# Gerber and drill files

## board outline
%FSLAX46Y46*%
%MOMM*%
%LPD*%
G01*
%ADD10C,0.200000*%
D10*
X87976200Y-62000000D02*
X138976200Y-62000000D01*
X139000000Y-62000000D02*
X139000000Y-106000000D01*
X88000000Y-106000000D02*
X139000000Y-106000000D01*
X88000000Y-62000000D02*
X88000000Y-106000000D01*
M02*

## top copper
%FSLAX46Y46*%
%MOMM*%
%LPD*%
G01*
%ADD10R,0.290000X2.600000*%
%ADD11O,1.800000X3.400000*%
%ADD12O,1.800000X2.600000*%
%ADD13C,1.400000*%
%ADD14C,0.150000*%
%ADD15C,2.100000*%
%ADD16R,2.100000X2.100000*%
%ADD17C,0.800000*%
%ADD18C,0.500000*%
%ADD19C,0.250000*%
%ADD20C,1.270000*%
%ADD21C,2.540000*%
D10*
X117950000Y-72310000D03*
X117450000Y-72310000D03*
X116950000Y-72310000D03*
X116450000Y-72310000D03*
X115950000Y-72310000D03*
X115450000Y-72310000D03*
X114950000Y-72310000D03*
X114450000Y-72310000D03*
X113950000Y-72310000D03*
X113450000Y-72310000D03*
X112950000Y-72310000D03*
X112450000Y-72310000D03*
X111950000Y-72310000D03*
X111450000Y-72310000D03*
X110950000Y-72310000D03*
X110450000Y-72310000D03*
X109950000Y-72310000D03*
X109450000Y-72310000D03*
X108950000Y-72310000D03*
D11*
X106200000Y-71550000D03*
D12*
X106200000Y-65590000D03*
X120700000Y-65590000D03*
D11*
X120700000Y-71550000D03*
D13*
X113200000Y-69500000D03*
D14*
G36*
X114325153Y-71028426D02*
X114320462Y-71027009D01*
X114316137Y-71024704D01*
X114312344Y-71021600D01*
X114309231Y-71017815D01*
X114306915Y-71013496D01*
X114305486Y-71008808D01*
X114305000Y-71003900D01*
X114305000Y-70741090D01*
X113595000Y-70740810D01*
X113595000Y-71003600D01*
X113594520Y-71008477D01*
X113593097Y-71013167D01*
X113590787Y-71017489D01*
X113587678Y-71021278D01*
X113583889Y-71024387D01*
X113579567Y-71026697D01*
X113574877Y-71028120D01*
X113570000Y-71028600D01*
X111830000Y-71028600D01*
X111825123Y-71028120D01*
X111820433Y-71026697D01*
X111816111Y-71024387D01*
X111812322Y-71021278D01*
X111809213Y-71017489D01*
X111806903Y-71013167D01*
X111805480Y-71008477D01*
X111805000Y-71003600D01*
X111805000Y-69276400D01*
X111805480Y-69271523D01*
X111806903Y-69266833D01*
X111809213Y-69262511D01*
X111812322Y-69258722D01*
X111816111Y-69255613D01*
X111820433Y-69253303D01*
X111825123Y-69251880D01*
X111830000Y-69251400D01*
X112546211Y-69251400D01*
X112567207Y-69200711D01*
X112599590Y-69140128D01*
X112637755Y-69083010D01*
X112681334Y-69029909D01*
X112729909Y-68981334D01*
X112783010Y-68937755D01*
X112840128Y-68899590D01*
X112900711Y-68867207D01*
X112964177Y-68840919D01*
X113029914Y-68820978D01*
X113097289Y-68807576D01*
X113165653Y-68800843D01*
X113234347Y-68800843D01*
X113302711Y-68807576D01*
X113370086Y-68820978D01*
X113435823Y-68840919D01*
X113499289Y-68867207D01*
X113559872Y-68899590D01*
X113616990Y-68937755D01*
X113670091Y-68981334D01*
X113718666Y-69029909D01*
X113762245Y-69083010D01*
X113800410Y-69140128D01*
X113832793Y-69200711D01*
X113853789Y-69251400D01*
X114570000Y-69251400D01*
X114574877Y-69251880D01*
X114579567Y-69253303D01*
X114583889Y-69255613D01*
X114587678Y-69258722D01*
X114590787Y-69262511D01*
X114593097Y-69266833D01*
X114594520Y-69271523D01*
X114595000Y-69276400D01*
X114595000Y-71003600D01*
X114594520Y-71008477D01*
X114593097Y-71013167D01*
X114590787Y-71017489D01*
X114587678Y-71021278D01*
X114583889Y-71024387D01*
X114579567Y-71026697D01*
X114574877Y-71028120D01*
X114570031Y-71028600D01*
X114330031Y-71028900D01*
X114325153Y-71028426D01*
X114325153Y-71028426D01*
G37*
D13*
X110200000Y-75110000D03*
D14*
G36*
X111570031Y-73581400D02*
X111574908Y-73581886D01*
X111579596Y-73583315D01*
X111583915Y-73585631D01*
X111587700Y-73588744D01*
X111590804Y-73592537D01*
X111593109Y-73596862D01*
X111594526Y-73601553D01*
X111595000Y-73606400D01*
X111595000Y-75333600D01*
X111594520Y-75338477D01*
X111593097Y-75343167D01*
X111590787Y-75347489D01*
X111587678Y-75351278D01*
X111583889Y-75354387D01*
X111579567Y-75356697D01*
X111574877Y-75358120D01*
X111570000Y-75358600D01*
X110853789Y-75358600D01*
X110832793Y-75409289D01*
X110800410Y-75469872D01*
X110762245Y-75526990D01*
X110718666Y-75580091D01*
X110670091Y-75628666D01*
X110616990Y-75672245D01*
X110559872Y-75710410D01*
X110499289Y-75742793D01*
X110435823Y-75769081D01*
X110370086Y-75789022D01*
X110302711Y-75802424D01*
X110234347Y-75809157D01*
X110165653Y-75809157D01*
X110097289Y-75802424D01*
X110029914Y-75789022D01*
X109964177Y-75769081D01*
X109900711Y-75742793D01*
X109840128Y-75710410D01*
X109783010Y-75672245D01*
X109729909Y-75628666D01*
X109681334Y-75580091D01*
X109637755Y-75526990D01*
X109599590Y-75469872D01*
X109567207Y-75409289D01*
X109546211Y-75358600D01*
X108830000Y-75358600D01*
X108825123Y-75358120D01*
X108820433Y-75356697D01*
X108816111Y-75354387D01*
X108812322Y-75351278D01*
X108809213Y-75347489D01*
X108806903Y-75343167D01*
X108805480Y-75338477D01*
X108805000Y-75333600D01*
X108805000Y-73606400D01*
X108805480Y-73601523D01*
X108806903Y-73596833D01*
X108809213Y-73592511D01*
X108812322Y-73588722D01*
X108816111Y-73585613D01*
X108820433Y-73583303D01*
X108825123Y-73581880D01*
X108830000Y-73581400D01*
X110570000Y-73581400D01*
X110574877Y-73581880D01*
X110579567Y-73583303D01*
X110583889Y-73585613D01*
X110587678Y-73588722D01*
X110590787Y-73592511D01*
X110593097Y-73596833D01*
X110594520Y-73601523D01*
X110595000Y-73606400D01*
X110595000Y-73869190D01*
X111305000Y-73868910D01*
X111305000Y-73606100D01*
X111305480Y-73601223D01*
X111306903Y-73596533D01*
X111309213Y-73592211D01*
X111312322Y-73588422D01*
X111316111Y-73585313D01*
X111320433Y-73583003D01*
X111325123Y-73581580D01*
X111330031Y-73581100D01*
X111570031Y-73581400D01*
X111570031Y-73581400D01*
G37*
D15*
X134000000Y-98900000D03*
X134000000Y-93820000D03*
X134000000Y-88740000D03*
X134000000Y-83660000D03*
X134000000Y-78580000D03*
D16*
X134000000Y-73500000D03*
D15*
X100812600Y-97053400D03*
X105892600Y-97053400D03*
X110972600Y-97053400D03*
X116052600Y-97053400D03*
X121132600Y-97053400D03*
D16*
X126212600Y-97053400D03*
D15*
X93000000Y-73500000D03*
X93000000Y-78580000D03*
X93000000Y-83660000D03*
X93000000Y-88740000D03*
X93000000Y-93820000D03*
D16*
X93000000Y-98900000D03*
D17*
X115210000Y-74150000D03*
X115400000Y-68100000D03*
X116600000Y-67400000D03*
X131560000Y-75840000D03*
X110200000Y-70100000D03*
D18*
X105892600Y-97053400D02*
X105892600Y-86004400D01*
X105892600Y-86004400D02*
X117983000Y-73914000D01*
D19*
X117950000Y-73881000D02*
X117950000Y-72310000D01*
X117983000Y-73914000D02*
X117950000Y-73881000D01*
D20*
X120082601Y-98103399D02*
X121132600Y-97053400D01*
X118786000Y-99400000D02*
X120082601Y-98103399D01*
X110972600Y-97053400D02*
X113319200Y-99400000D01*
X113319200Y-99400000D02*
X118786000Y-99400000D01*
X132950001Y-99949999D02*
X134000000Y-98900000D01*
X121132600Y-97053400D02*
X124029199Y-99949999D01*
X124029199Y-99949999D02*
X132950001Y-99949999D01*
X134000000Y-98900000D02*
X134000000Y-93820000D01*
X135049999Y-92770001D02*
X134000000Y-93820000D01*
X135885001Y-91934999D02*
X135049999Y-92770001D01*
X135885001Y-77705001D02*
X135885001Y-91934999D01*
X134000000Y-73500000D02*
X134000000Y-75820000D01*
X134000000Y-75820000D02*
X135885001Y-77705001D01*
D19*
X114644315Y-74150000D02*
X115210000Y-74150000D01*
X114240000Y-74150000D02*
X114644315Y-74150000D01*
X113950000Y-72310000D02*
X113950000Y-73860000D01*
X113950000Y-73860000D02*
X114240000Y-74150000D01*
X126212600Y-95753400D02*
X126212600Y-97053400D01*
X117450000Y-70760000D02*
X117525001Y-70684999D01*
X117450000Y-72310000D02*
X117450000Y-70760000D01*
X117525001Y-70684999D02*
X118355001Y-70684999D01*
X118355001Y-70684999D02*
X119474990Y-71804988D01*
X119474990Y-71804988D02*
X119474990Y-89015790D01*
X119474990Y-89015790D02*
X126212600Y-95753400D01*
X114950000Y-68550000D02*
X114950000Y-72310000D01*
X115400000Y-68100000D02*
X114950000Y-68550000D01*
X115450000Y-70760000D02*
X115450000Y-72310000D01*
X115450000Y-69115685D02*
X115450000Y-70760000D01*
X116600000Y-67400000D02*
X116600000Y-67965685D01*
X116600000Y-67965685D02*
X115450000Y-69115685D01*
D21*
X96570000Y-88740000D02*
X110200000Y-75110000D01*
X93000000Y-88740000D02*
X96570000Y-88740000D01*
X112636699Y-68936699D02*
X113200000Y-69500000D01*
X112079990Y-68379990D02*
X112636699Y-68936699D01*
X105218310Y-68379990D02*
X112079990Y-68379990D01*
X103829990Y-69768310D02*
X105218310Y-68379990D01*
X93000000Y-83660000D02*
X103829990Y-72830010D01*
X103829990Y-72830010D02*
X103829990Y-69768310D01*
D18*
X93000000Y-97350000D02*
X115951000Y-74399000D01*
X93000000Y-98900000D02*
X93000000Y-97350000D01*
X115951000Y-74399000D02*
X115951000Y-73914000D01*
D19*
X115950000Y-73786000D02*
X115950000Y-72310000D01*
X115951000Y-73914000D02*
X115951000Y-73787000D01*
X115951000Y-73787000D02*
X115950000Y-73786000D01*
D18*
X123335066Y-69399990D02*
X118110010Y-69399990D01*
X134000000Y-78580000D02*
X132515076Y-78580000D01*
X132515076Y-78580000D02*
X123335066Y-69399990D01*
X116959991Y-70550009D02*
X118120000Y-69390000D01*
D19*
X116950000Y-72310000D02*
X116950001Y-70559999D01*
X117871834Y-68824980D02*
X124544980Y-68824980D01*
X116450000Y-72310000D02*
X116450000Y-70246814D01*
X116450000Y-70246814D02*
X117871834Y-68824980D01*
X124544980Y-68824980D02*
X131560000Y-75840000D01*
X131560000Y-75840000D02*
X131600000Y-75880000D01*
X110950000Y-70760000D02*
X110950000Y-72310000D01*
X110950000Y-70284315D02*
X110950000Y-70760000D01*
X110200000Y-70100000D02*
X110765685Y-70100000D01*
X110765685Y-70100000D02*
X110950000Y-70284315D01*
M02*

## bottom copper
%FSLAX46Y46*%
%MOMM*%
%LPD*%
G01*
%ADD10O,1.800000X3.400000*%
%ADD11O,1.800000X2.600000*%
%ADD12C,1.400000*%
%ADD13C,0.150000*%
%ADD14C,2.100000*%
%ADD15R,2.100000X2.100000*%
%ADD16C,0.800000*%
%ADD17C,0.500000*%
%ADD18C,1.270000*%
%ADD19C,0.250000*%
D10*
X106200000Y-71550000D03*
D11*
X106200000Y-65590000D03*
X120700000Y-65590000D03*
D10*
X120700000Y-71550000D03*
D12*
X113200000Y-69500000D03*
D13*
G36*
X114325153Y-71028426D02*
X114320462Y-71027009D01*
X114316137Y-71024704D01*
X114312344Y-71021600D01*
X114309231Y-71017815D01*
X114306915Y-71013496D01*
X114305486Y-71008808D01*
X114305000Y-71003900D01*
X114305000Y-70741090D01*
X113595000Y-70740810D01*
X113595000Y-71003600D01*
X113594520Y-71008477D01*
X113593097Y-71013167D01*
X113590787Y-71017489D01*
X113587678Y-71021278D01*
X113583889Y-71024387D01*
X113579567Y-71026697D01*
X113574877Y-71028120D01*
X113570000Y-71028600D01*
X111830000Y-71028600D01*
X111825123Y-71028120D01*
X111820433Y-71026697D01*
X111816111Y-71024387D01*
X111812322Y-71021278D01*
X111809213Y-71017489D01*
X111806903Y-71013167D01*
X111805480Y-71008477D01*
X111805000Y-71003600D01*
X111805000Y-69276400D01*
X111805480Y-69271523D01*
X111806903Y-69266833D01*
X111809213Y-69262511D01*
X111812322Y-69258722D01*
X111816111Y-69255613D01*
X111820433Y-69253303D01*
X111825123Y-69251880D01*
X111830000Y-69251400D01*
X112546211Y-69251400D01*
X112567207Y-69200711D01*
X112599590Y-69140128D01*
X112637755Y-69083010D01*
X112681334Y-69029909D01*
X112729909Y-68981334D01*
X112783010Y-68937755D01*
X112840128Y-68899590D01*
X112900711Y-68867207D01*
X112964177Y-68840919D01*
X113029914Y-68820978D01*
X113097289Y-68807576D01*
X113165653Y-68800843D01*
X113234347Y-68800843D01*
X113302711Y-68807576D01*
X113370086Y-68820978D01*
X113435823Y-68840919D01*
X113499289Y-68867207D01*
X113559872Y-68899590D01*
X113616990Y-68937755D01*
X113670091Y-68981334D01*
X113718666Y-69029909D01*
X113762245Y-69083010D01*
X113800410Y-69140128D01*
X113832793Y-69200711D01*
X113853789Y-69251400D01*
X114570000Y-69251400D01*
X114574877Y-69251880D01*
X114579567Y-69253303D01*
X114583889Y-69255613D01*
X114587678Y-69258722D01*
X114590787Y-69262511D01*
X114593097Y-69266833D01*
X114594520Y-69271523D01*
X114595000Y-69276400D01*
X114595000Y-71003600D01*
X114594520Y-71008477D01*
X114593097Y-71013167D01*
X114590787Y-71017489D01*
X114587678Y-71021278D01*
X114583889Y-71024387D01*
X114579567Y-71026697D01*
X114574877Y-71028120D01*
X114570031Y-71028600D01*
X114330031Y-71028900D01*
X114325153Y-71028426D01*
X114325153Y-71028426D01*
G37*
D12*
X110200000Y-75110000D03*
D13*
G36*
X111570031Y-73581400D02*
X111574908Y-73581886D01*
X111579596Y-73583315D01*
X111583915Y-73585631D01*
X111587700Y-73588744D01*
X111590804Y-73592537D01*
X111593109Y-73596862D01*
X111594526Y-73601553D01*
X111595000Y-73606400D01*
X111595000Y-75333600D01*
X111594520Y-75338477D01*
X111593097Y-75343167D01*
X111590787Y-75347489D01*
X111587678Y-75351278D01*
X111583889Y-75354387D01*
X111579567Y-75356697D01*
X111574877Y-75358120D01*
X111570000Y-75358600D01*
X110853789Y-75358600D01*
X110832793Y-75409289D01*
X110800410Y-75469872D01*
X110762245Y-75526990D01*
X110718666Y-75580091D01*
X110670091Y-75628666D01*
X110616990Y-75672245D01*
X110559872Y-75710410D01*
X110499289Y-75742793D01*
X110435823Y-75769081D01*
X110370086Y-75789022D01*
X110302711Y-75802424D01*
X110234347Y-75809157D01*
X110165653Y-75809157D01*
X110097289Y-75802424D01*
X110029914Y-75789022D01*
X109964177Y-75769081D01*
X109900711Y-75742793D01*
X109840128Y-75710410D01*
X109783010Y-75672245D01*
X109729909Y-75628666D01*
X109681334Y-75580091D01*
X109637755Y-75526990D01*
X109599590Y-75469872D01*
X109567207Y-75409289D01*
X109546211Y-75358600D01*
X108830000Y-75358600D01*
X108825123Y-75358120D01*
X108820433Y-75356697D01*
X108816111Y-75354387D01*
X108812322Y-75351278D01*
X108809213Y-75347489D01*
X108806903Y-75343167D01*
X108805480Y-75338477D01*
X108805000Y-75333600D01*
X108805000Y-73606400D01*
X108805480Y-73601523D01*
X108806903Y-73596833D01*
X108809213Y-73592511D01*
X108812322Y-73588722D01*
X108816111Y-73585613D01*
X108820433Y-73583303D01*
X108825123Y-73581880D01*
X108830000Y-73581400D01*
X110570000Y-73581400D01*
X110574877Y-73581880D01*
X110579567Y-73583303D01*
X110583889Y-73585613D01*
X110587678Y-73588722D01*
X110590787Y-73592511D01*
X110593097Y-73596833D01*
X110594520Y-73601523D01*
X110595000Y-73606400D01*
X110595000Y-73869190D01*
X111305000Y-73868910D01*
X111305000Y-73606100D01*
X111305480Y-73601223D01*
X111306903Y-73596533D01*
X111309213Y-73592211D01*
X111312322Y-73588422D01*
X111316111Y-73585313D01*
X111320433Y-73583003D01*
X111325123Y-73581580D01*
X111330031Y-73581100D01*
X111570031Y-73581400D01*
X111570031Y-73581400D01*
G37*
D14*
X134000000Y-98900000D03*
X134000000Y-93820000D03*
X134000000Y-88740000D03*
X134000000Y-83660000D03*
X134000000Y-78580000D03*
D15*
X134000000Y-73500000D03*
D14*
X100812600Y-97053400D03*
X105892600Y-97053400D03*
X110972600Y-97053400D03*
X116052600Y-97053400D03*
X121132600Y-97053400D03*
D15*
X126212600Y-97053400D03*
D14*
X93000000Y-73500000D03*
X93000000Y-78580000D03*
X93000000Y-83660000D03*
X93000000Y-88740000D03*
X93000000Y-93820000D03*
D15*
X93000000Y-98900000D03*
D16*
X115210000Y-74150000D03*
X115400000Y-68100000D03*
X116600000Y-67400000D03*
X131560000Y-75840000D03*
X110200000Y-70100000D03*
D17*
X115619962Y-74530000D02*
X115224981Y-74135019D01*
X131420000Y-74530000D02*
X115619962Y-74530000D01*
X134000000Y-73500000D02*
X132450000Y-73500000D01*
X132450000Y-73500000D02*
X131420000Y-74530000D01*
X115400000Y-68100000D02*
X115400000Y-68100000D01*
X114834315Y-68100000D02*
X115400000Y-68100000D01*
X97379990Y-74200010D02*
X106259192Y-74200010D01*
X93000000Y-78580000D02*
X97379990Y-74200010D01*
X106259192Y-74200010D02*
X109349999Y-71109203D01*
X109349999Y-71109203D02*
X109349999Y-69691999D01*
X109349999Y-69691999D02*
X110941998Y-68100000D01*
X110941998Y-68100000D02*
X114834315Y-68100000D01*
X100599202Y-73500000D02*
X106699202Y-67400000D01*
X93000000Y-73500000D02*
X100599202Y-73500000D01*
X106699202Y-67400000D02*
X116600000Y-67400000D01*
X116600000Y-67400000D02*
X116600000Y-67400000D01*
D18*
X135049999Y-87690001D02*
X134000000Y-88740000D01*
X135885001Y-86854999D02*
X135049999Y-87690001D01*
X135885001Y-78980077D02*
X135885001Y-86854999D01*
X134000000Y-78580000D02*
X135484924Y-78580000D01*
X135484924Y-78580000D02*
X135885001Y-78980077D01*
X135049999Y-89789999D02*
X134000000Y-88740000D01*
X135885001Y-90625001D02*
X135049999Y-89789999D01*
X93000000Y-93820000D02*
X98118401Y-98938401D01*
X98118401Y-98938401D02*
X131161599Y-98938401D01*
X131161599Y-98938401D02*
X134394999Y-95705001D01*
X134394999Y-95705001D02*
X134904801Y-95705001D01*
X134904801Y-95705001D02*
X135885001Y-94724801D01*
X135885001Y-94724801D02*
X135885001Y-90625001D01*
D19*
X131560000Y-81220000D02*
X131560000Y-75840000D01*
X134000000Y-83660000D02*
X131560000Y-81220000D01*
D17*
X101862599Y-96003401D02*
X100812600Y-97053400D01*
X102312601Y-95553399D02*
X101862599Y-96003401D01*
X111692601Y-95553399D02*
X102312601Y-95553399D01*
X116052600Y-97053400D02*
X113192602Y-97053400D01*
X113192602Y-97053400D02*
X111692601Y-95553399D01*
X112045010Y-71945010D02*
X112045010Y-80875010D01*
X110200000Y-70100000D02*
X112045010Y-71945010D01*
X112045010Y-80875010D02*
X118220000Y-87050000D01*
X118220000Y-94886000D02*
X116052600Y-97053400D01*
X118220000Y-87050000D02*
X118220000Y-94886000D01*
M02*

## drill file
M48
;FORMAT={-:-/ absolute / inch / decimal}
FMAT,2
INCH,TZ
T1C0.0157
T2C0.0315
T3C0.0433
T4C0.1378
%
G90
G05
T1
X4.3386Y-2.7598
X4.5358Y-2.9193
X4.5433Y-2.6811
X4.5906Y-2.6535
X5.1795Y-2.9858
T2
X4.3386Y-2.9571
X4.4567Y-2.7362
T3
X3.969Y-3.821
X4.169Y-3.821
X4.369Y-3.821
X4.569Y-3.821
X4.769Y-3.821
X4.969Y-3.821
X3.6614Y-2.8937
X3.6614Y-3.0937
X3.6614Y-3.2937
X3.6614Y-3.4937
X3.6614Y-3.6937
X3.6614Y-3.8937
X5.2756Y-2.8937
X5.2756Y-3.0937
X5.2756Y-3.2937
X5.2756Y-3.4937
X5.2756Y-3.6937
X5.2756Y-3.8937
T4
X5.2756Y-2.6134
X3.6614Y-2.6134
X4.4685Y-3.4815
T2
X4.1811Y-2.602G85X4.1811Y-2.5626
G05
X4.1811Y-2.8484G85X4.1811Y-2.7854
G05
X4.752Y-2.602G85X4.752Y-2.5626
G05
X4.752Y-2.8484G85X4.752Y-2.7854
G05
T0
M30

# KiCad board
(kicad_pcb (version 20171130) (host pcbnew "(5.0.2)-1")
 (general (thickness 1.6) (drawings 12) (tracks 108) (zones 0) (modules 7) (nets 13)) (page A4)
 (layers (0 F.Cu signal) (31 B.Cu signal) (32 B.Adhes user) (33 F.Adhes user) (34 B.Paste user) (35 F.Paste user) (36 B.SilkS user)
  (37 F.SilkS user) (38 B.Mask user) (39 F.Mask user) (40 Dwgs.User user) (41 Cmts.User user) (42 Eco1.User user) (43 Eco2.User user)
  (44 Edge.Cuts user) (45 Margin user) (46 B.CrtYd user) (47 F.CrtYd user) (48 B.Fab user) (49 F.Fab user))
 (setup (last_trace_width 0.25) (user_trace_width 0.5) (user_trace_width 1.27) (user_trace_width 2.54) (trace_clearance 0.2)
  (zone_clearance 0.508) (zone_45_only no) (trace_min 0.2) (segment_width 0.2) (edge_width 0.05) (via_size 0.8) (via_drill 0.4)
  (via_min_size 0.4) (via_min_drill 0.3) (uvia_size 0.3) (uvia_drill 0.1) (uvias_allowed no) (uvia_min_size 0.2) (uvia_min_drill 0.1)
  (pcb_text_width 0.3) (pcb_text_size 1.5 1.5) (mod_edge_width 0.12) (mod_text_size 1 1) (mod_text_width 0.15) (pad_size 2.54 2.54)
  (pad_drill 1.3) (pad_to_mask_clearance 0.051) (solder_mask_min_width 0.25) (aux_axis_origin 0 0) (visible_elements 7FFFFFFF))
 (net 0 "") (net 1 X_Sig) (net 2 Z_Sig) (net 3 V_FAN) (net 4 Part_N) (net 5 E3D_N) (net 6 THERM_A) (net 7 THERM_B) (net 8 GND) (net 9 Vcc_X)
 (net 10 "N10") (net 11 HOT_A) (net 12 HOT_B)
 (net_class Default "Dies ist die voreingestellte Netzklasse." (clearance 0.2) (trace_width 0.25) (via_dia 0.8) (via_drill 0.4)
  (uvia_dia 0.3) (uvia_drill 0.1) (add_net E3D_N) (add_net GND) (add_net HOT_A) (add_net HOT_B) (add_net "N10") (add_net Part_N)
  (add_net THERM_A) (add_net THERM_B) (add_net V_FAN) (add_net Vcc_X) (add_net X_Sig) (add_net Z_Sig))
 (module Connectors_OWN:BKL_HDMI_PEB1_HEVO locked (layer F.Cu) (at 120.7 62 180)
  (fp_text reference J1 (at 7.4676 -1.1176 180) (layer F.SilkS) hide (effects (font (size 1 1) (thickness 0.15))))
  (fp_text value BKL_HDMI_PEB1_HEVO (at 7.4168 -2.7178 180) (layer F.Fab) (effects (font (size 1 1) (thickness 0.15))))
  (pad 19 smd rect (at 2.75 -10.31 180) (size 0.29 2.6) (layers F.Cu F.Paste F.Mask) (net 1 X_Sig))
  (pad 18 smd rect (at 3.25 -10.31 180) (size 0.29 2.6) (layers F.Cu F.Paste F.Mask) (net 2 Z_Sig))
  (pad 17 smd rect (at 3.75 -10.31 180) (size 0.29 2.6) (layers F.Cu F.Paste F.Mask) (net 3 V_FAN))
  (pad 16 smd rect (at 4.25 -10.31 180) (size 0.29 2.6) (layers F.Cu F.Paste F.Mask) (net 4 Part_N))
  (pad 15 smd rect (at 4.75 -10.31 180) (size 0.29 2.6) (layers F.Cu F.Paste F.Mask) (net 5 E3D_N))
  (pad 14 smd rect (at 5.25 -10.31 180) (size 0.29 2.6) (layers F.Cu F.Paste F.Mask) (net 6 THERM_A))
  (pad 13 smd rect (at 5.75 -10.31 180) (size 0.29 2.6) (layers F.Cu F.Paste F.Mask) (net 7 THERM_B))
  (pad "" smd rect (at 6.25 -10.31 180) (size 0.29 2.6) (layers F.Cu F.Paste F.Mask))
  (pad 11 smd rect (at 6.75 -10.31 180) (size 0.29 2.6) (layers F.Cu F.Paste F.Mask) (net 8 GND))
  (pad "" smd rect (at 7.25 -10.31 180) (size 0.29 2.6) (layers F.Cu F.Paste F.Mask))
  (pad "" smd rect (at 7.75 -10.31 180) (size 0.29 2.6) (layers F.Cu F.Paste F.Mask))
  (pad "" smd rect (at 8.25 -10.31 180) (size 0.29 2.6) (layers F.Cu F.Paste F.Mask))
  (pad "" smd rect (at 8.75 -10.31 180) (size 0.29 2.6) (layers F.Cu F.Paste F.Mask))
  (pad "" smd rect (at 9.25 -10.31 180) (size 0.29 2.6) (layers F.Cu F.Paste F.Mask))
  (pad 5 smd rect (at 9.75 -10.31 180) (size 0.29 2.6) (layers F.Cu F.Paste F.Mask) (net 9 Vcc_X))
  (pad "" smd rect (at 10.25 -10.31 180) (size 0.29 2.6) (layers F.Cu F.Paste F.Mask))
  (pad "" smd rect (at 10.75 -10.31 180) (size 0.29 2.6) (layers F.Cu F.Paste F.Mask))
  (pad "" smd rect (at 11.25 -10.31 180) (size 0.29 2.6) (layers F.Cu F.Paste F.Mask))
  (pad "" smd rect (at 11.75 -10.31 180) (size 0.29 2.6) (layers F.Cu F.Paste F.Mask))
  (pad SH thru_hole oval (at 14.5 -9.55 180) (size 1.8 3.4) (drill oval 0.8 2.4) (layers *.Cu *.Mask) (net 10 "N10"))
  (pad SH thru_hole oval (at 14.5 -3.59 180) (size 1.8 2.6) (drill oval 0.8 1.8) (layers *.Cu *.Mask) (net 10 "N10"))
  (pad SH thru_hole oval (at 0 -3.59 180) (size 1.8 2.6) (drill oval 0.8 1.8) (layers *.Cu *.Mask) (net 10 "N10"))
  (pad SH thru_hole oval (at 0 -9.55 180) (size 1.8 3.4) (drill oval 0.8 2.4) (layers *.Cu *.Mask) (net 10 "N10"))
  (pad 7 thru_hole custom (at 7.5 -7.5 180) (size 1.4 1.4) (drill 0.8) (layers *.Cu *.Mask) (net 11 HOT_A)
   (options (clearance outline) (anchor circle)) (primitives))
  (pad 1 thru_hole custom (at 10.5 -13.11) (size 1.4 1.4) (drill 0.8) (layers *.Cu *.Mask) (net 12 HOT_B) (zone_connect 0)
   (options (clearance outline) (anchor circle)) (primitives)))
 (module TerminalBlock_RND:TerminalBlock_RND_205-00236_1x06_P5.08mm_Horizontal (layer F.Cu) (at 134 73.5 270)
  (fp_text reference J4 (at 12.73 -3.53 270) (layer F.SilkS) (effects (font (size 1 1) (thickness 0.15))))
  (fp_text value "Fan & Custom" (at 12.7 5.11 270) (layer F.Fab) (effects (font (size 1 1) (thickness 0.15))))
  (pad 6 thru_hole circle (at 25.4 0 270) (size 2.1 2.1) (drill 1.1) (layers *.Cu *.Mask) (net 8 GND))
  (pad 5 thru_hole circle (at 20.32 0 270) (size 2.1 2.1) (drill 1.1) (layers *.Cu *.Mask) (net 8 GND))
  (pad 4 thru_hole circle (at 15.24 0 270) (size 2.1 2.1) (drill 1.1) (layers *.Cu *.Mask) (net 3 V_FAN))
  (pad 3 thru_hole circle (at 10.16 0 270) (size 2.1 2.1) (drill 1.1) (layers *.Cu *.Mask) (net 4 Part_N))
  (pad 2 thru_hole circle (at 5.08 0 270) (size 2.1 2.1) (drill 1.1) (layers *.Cu *.Mask) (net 3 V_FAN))
  (pad 1 thru_hole rect (at 0 0 270) (size 2.1 2.1) (drill 1.1) (layers *.Cu *.Mask) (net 8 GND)))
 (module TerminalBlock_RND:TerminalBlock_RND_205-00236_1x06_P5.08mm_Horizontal (layer F.Cu) (at 126.2126 97.0534 180)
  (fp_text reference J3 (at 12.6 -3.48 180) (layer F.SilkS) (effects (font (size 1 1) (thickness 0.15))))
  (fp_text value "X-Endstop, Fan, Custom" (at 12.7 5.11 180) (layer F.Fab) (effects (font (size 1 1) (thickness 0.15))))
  (pad 6 thru_hole circle (at 25.4 0 180) (size 2.1 2.1) (drill 1.1) (layers *.Cu *.Mask) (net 9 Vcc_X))
  (pad 5 thru_hole circle (at 20.32 0 180) (size 2.1 2.1) (drill 1.1) (layers *.Cu *.Mask) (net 1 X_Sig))
  (pad 4 thru_hole circle (at 15.24 0 180) (size 2.1 2.1) (drill 1.1) (layers *.Cu *.Mask) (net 8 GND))
  (pad 3 thru_hole circle (at 10.16 0 180) (size 2.1 2.1) (drill 1.1) (layers *.Cu *.Mask) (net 9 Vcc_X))
  (pad 2 thru_hole circle (at 5.08 0 180) (size 2.1 2.1) (drill 1.1) (layers *.Cu *.Mask) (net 8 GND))
  (pad 1 thru_hole rect (at 0 0 180) (size 2.1 2.1) (drill 1.1) (layers *.Cu *.Mask) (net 2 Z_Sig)))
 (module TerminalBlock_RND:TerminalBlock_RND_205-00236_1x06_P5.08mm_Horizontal (layer F.Cu) (at 93 98.9 90)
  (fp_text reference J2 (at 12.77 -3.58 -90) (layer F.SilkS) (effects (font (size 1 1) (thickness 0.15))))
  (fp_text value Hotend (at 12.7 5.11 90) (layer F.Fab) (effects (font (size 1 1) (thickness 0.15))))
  (pad 6 thru_hole circle (at 25.4 0 90) (size 2.1 2.1) (drill 1.1) (layers *.Cu *.Mask) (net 6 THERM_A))
  (pad 5 thru_hole circle (at 20.32 0 90) (size 2.1 2.1) (drill 1.1) (layers *.Cu *.Mask) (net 7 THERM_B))
  (pad 4 thru_hole circle (at 15.24 0 90) (size 2.1 2.1) (drill 1.1) (layers *.Cu *.Mask) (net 11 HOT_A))
  (pad 3 thru_hole circle (at 10.16 0 90) (size 2.1 2.1) (drill 1.1) (layers *.Cu *.Mask) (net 12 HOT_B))
  (pad 2 thru_hole circle (at 5.08 0 90) (size 2.1 2.1) (drill 1.1) (layers *.Cu *.Mask) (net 3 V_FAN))
  (pad 1 thru_hole rect (at 0 0 90) (size 2.1 2.1) (drill 1.1) (layers *.Cu *.Mask) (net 5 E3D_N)))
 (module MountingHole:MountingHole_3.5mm (layer F.Cu) (at 113.5 88.43)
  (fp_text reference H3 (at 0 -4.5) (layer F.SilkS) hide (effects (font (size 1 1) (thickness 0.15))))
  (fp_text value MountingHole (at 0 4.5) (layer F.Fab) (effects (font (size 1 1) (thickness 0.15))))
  (pad 1 np_thru_hole circle (at 0 0) (size 3.5 3.5) (drill 3.5) (layers *.Cu *.Mask)))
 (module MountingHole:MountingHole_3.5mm (layer F.Cu) (at 134 66.38)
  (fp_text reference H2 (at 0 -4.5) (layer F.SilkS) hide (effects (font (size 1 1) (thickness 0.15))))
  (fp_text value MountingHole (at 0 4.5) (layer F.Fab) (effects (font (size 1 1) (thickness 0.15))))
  (pad 1 np_thru_hole circle (at 0 0) (size 3.5 3.5) (drill 3.5) (layers *.Cu *.Mask)))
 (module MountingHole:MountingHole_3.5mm (layer F.Cu) (at 93 66.38)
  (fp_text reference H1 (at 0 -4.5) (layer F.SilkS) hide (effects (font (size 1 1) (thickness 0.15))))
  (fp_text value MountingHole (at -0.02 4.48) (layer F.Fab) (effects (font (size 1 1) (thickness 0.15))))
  (pad 1 np_thru_hole circle (at 0 0) (size 3.5 3.5) (drill 3.5) (layers *.Cu *.Mask)))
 (gr_line (start 87.9762 62) (end 138.9762 62) (layer Edge.Cuts) (width 0.2))
 (gr_line (start 139 62) (end 139 106) (layer Edge.Cuts) (width 0.2))
 (gr_line (start 88 106) (end 139 106) (layer Edge.Cuts) (width 0.2))
 (gr_line (start 88 62) (end 88 106) (layer Edge.Cuts) (width 0.2))
 (segment (start 105.8926 97.0534) (end 105.8926 86.0044) (width 0.5) (layer F.Cu) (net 1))
 (segment (start 105.8926 86.0044) (end 117.983 73.914) (width 0.5) (layer F.Cu) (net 1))
 (segment (start 117.95 73.881) (end 117.95 72.31) (width 0.25) (layer F.Cu) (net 1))
 (segment (start 117.983 73.914) (end 117.95 73.881) (width 0.25) (layer F.Cu) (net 1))
 (via (at 115.21 74.15) (size 0.8) (drill 0.4) (layers F.Cu B.Cu) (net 8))
 (segment (start 120.082601 98.103399) (end 121.1326 97.0534) (width 1.27) (layer F.Cu) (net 8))
 (segment (start 118.786 99.4) (end 120.082601 98.103399) (width 1.27) (layer F.Cu) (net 8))
 (segment (start 110.9726 97.0534) (end 113.3192 99.4) (width 1.27) (layer F.Cu) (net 8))
 (segment (start 113.3192 99.4) (end 118.786 99.4) (width 1.27) (layer F.Cu) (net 8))
 (segment (start 132.950001 99.949999) (end 134 98.9) (width 1.27) (layer F.Cu) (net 8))
 (segment (start 121.1326 97.0534) (end 124.029199 99.949999) (width 1.27) (layer F.Cu) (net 8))
 (segment (start 124.029199 99.949999) (end 132.950001 99.949999) (width 1.27) (layer F.Cu) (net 8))
 (segment (start 134 98.9) (end 134 93.82) (width 1.27) (layer F.Cu) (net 8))
 (segment (start 135.049999 92.770001) (end 134 93.82) (width 1.27) (layer F.Cu) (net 8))
 (segment (start 135.885001 91.934999) (end 135.049999 92.770001) (width 1.27) (layer F.Cu) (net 8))
 (segment (start 135.885001 77.705001) (end 135.885001 91.934999) (width 1.27) (layer F.Cu) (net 8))
 (segment (start 134 73.5) (end 134 75.82) (width 1.27) (layer F.Cu) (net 8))
 (segment (start 134 75.82) (end 135.885001 77.705001) (width 1.27) (layer F.Cu) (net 8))
 (segment (start 114.644315 74.15) (end 115.21 74.15) (width 0.25) (layer F.Cu) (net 8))
 (segment (start 114.24 74.15) (end 114.644315 74.15) (width 0.25) (layer F.Cu) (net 8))
 (segment (start 113.95 72.31) (end 113.95 73.86) (width 0.25) (layer F.Cu) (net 8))
 (segment (start 113.95 73.86) (end 114.24 74.15) (width 0.25) (layer F.Cu) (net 8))
 (segment (start 115.619962 74.53) (end 115.224981 74.135019) (width 0.5) (layer B.Cu) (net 8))
 (segment (start 131.42 74.53) (end 115.619962 74.53) (width 0.5) (layer B.Cu) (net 8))
 (segment (start 134 73.5) (end 132.45 73.5) (width 0.5) (layer B.Cu) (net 8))
 (segment (start 132.45 73.5) (end 131.42 74.53) (width 0.5) (layer B.Cu) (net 8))
 (segment (start 126.2126 95.7534) (end 126.2126 97.0534) (width 0.25) (layer F.Cu) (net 2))
 (segment (start 117.45 70.76) (end 117.525001 70.684999) (width 0.25) (layer F.Cu) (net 2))
 (segment (start 117.45 72.31) (end 117.45 70.76) (width 0.25) (layer F.Cu) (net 2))
 (segment (start 117.525001 70.684999) (end 118.355001 70.684999) (width 0.25) (layer F.Cu) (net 2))
 (segment (start 118.355001 70.684999) (end 119.47499 71.804988) (width 0.25) (layer F.Cu) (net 2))
 (segment (start 119.47499 71.804988) (end 119.47499 89.01579) (width 0.25) (layer F.Cu) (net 2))
 (segment (start 119.47499 89.01579) (end 126.2126 95.7534) (width 0.25) (layer F.Cu) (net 2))
 (segment (start 115.4 68.1) (end 115.4 68.1) (width 0.5) (layer B.Cu) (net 7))
 (via (at 115.4 68.1) (size 0.8) (drill 0.4) (layers F.Cu B.Cu) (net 7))
 (segment (start 114.95 68.55) (end 114.95 72.31) (width 0.25) (layer F.Cu) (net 7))
 (segment (start 115.4 68.1) (end 114.95 68.55) (width 0.25) (layer F.Cu) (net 7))
 (segment (start 114.834315 68.1) (end 115.4 68.1) (width 0.5) (layer B.Cu) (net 7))
 (segment (start 97.37999 74.20001) (end 106.259192 74.20001) (width 0.5) (layer B.Cu) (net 7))
 (segment (start 93 78.58) (end 97.37999 74.20001) (width 0.5) (layer B.Cu) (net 7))
 (segment (start 106.259192 74.20001) (end 109.349999 71.109203) (width 0.5) (layer B.Cu) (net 7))
 (segment (start 109.349999 71.109203) (end 109.349999 69.691999) (width 0.5) (layer B.Cu) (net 7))
 (segment (start 109.349999 69.691999) (end 110.941998 68.1) (width 0.5) (layer B.Cu) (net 7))
 (segment (start 110.941998 68.1) (end 114.834315 68.1) (width 0.5) (layer B.Cu) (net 7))
 (segment (start 100.599202 73.5) (end 106.699202 67.4) (width 0.5) (layer B.Cu) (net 6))
 (segment (start 93 73.5) (end 100.599202 73.5) (width 0.5) (layer B.Cu) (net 6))
 (segment (start 106.699202 67.4) (end 116.6 67.4) (width 0.5) (layer B.Cu) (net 6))
 (segment (start 116.6 67.4) (end 116.6 67.4) (width 0.5) (layer B.Cu) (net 6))
 (via (at 116.6 67.4) (size 0.8) (drill 0.4) (layers F.Cu B.Cu) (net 6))
 (segment (start 115.45 70.76) (end 115.45 72.31) (width 0.25) (layer F.Cu) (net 6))
 (segment (start 115.45 69.115685) (end 115.45 70.76) (width 0.25) (layer F.Cu) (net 6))
 (segment (start 116.6 67.4) (end 116.6 67.965685) (width 0.25) (layer F.Cu) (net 6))
 (segment (start 116.6 67.965685) (end 115.45 69.115685) (width 0.25) (layer F.Cu) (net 6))
 (segment (start 96.57 88.74) (end 110.2 75.11) (width 2.54) (layer F.Cu) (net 12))
 (segment (start 93 88.74) (end 96.57 88.74) (width 2.54) (layer F.Cu) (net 12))
 (segment (start 112.636699 68.936699) (end 113.2 69.5) (width 2.54) (layer F.Cu) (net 11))
 (segment (start 112.07999 68.37999) (end 112.636699 68.936699) (width 2.54) (layer F.Cu) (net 11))
 (segment (start 105.21831 68.37999) (end 112.07999 68.37999) (width 2.54) (layer F.Cu) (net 11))
 (segment (start 103.82999 69.76831) (end 105.21831 68.37999) (width 2.54) (layer F.Cu) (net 11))
 (segment (start 93 83.66) (end 103.82999 72.83001) (width 2.54) (layer F.Cu) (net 11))
 (segment (start 103.82999 72.83001) (end 103.82999 69.76831) (width 2.54) (layer F.Cu) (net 11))
 (segment (start 93 97.35) (end 115.951 74.399) (width 0.5) (layer F.Cu) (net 5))
 (segment (start 93 98.9) (end 93 97.35) (width 0.5) (layer F.Cu) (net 5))
 (segment (start 115.951 74.399) (end 115.951 73.914) (width 0.5) (layer F.Cu) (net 5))
 (segment (start 115.95 73.786) (end 115.95 72.31) (width 0.25) (layer F.Cu) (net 5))
 (segment (start 115.951 73.914) (end 115.951 73.787) (width 0.25) (layer F.Cu) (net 5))
 (segment (start 115.951 73.787) (end 115.95 73.786) (width 0.25) (layer F.Cu) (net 5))
 (segment (start 135.049999 87.690001) (end 134 88.74) (width 1.27) (layer B.Cu) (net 3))
 (segment (start 135.885001 86.854999) (end 135.049999 87.690001) (width 1.27) (layer B.Cu) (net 3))
 (segment (start 135.885001 78.980077) (end 135.885001 86.854999) (width 1.27) (layer B.Cu) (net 3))
 (segment (start 134 78.58) (end 135.484924 78.58) (width 1.27) (layer B.Cu) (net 3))
 (segment (start 135.484924 78.58) (end 135.885001 78.980077) (width 1.27) (layer B.Cu) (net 3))
 (segment (start 135.049999 89.789999) (end 134 88.74) (width 1.27) (layer B.Cu) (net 3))
 (segment (start 135.885001 90.625001) (end 135.049999 89.789999) (width 1.27) (layer B.Cu) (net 3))
 (segment (start 93 93.82) (end 98.118401 98.938401) (width 1.27) (layer B.Cu) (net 3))
 (segment (start 98.118401 98.938401) (end 131.161599 98.938401) (width 1.27) (layer B.Cu) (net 3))
 (segment (start 131.161599 98.938401) (end 134.394999 95.705001) (width 1.27) (layer B.Cu) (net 3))
 (segment (start 134.394999 95.705001) (end 134.904801 95.705001) (width 1.27) (layer B.Cu) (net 3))
 (segment (start 134.904801 95.705001) (end 135.885001 94.724801) (width 1.27) (layer B.Cu) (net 3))
 (segment (start 135.885001 94.724801) (end 135.885001 90.625001) (width 1.27) (layer B.Cu) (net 3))
 (segment (start 123.335066 69.39999) (end 118.11001 69.39999) (width 0.5) (layer F.Cu) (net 3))
 (segment (start 134 78.58) (end 132.515076 78.58) (width 0.5) (layer F.Cu) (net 3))
 (segment (start 132.515076 78.58) (end 123.335066 69.39999) (width 0.5) (layer F.Cu) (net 3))
 (segment (start 116.959991 70.550009) (end 118.12 69.39) (width 0.5) (layer F.Cu) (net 3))
 (segment (start 116.95 72.31) (end 116.950001 70.559999) (width 0.25) (layer F.Cu) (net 3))
 (segment (start 117.871834 68.82498) (end 124.54498 68.82498) (width 0.25) (layer F.Cu) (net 4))
 (segment (start 116.45 72.31) (end 116.45 70.246814) (width 0.25) (layer F.Cu) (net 4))
 (segment (start 116.45 70.246814) (end 117.871834 68.82498) (width 0.25) (layer F.Cu) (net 4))
 (segment (start 124.54498 68.82498) (end 131.56 75.84) (width 0.25) (layer F.Cu) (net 4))
 (segment (start 131.56 75.84) (end 131.6 75.88) (width 0.25) (layer F.Cu) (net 4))
 (via (at 131.56 75.84) (size 0.8) (drill 0.4) (layers F.Cu B.Cu) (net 4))
 (segment (start 131.56 81.22) (end 131.56 75.84) (width 0.25) (layer B.Cu) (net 4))
 (segment (start 134 83.66) (end 131.56 81.22) (width 0.25) (layer B.Cu) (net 4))
 (via (at 110.2 70.1) (size 0.8) (drill 0.4) (layers F.Cu B.Cu) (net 9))
 (segment (start 110.95 70.76) (end 110.95 72.31) (width 0.25) (layer F.Cu) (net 9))
 (segment (start 110.95 70.284315) (end 110.95 70.76) (width 0.25) (layer F.Cu) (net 9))
 (segment (start 110.2 70.1) (end 110.765685 70.1) (width 0.25) (layer F.Cu) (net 9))
 (segment (start 110.765685 70.1) (end 110.95 70.284315) (width 0.25) (layer F.Cu) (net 9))
 (segment (start 101.862599 96.003401) (end 100.8126 97.0534) (width 0.5) (layer B.Cu) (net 9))
 (segment (start 102.312601 95.553399) (end 101.862599 96.003401) (width 0.5) (layer B.Cu) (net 9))
 (segment (start 111.692601 95.553399) (end 102.312601 95.553399) (width 0.5) (layer B.Cu) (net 9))
 (segment (start 116.0526 97.0534) (end 113.192602 97.0534) (width 0.5) (layer B.Cu) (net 9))
 (segment (start 113.192602 97.0534) (end 111.692601 95.553399) (width 0.5) (layer B.Cu) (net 9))
 (segment (start 112.04501 71.94501) (end 112.04501 80.87501) (width 0.5) (layer B.Cu) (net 9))
 (segment (start 110.2 70.1) (end 112.04501 71.94501) (width 0.5) (layer B.Cu) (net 9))
 (segment (start 112.04501 80.87501) (end 118.22 87.05) (width 0.5) (layer B.Cu) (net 9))
 (segment (start 118.22 94.886) (end 116.0526 97.0534) (width 0.5) (layer B.Cu) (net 9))
 (segment (start 118.22 87.05) (end 118.22 94.886) (width 0.5) (layer B.Cu) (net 9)))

